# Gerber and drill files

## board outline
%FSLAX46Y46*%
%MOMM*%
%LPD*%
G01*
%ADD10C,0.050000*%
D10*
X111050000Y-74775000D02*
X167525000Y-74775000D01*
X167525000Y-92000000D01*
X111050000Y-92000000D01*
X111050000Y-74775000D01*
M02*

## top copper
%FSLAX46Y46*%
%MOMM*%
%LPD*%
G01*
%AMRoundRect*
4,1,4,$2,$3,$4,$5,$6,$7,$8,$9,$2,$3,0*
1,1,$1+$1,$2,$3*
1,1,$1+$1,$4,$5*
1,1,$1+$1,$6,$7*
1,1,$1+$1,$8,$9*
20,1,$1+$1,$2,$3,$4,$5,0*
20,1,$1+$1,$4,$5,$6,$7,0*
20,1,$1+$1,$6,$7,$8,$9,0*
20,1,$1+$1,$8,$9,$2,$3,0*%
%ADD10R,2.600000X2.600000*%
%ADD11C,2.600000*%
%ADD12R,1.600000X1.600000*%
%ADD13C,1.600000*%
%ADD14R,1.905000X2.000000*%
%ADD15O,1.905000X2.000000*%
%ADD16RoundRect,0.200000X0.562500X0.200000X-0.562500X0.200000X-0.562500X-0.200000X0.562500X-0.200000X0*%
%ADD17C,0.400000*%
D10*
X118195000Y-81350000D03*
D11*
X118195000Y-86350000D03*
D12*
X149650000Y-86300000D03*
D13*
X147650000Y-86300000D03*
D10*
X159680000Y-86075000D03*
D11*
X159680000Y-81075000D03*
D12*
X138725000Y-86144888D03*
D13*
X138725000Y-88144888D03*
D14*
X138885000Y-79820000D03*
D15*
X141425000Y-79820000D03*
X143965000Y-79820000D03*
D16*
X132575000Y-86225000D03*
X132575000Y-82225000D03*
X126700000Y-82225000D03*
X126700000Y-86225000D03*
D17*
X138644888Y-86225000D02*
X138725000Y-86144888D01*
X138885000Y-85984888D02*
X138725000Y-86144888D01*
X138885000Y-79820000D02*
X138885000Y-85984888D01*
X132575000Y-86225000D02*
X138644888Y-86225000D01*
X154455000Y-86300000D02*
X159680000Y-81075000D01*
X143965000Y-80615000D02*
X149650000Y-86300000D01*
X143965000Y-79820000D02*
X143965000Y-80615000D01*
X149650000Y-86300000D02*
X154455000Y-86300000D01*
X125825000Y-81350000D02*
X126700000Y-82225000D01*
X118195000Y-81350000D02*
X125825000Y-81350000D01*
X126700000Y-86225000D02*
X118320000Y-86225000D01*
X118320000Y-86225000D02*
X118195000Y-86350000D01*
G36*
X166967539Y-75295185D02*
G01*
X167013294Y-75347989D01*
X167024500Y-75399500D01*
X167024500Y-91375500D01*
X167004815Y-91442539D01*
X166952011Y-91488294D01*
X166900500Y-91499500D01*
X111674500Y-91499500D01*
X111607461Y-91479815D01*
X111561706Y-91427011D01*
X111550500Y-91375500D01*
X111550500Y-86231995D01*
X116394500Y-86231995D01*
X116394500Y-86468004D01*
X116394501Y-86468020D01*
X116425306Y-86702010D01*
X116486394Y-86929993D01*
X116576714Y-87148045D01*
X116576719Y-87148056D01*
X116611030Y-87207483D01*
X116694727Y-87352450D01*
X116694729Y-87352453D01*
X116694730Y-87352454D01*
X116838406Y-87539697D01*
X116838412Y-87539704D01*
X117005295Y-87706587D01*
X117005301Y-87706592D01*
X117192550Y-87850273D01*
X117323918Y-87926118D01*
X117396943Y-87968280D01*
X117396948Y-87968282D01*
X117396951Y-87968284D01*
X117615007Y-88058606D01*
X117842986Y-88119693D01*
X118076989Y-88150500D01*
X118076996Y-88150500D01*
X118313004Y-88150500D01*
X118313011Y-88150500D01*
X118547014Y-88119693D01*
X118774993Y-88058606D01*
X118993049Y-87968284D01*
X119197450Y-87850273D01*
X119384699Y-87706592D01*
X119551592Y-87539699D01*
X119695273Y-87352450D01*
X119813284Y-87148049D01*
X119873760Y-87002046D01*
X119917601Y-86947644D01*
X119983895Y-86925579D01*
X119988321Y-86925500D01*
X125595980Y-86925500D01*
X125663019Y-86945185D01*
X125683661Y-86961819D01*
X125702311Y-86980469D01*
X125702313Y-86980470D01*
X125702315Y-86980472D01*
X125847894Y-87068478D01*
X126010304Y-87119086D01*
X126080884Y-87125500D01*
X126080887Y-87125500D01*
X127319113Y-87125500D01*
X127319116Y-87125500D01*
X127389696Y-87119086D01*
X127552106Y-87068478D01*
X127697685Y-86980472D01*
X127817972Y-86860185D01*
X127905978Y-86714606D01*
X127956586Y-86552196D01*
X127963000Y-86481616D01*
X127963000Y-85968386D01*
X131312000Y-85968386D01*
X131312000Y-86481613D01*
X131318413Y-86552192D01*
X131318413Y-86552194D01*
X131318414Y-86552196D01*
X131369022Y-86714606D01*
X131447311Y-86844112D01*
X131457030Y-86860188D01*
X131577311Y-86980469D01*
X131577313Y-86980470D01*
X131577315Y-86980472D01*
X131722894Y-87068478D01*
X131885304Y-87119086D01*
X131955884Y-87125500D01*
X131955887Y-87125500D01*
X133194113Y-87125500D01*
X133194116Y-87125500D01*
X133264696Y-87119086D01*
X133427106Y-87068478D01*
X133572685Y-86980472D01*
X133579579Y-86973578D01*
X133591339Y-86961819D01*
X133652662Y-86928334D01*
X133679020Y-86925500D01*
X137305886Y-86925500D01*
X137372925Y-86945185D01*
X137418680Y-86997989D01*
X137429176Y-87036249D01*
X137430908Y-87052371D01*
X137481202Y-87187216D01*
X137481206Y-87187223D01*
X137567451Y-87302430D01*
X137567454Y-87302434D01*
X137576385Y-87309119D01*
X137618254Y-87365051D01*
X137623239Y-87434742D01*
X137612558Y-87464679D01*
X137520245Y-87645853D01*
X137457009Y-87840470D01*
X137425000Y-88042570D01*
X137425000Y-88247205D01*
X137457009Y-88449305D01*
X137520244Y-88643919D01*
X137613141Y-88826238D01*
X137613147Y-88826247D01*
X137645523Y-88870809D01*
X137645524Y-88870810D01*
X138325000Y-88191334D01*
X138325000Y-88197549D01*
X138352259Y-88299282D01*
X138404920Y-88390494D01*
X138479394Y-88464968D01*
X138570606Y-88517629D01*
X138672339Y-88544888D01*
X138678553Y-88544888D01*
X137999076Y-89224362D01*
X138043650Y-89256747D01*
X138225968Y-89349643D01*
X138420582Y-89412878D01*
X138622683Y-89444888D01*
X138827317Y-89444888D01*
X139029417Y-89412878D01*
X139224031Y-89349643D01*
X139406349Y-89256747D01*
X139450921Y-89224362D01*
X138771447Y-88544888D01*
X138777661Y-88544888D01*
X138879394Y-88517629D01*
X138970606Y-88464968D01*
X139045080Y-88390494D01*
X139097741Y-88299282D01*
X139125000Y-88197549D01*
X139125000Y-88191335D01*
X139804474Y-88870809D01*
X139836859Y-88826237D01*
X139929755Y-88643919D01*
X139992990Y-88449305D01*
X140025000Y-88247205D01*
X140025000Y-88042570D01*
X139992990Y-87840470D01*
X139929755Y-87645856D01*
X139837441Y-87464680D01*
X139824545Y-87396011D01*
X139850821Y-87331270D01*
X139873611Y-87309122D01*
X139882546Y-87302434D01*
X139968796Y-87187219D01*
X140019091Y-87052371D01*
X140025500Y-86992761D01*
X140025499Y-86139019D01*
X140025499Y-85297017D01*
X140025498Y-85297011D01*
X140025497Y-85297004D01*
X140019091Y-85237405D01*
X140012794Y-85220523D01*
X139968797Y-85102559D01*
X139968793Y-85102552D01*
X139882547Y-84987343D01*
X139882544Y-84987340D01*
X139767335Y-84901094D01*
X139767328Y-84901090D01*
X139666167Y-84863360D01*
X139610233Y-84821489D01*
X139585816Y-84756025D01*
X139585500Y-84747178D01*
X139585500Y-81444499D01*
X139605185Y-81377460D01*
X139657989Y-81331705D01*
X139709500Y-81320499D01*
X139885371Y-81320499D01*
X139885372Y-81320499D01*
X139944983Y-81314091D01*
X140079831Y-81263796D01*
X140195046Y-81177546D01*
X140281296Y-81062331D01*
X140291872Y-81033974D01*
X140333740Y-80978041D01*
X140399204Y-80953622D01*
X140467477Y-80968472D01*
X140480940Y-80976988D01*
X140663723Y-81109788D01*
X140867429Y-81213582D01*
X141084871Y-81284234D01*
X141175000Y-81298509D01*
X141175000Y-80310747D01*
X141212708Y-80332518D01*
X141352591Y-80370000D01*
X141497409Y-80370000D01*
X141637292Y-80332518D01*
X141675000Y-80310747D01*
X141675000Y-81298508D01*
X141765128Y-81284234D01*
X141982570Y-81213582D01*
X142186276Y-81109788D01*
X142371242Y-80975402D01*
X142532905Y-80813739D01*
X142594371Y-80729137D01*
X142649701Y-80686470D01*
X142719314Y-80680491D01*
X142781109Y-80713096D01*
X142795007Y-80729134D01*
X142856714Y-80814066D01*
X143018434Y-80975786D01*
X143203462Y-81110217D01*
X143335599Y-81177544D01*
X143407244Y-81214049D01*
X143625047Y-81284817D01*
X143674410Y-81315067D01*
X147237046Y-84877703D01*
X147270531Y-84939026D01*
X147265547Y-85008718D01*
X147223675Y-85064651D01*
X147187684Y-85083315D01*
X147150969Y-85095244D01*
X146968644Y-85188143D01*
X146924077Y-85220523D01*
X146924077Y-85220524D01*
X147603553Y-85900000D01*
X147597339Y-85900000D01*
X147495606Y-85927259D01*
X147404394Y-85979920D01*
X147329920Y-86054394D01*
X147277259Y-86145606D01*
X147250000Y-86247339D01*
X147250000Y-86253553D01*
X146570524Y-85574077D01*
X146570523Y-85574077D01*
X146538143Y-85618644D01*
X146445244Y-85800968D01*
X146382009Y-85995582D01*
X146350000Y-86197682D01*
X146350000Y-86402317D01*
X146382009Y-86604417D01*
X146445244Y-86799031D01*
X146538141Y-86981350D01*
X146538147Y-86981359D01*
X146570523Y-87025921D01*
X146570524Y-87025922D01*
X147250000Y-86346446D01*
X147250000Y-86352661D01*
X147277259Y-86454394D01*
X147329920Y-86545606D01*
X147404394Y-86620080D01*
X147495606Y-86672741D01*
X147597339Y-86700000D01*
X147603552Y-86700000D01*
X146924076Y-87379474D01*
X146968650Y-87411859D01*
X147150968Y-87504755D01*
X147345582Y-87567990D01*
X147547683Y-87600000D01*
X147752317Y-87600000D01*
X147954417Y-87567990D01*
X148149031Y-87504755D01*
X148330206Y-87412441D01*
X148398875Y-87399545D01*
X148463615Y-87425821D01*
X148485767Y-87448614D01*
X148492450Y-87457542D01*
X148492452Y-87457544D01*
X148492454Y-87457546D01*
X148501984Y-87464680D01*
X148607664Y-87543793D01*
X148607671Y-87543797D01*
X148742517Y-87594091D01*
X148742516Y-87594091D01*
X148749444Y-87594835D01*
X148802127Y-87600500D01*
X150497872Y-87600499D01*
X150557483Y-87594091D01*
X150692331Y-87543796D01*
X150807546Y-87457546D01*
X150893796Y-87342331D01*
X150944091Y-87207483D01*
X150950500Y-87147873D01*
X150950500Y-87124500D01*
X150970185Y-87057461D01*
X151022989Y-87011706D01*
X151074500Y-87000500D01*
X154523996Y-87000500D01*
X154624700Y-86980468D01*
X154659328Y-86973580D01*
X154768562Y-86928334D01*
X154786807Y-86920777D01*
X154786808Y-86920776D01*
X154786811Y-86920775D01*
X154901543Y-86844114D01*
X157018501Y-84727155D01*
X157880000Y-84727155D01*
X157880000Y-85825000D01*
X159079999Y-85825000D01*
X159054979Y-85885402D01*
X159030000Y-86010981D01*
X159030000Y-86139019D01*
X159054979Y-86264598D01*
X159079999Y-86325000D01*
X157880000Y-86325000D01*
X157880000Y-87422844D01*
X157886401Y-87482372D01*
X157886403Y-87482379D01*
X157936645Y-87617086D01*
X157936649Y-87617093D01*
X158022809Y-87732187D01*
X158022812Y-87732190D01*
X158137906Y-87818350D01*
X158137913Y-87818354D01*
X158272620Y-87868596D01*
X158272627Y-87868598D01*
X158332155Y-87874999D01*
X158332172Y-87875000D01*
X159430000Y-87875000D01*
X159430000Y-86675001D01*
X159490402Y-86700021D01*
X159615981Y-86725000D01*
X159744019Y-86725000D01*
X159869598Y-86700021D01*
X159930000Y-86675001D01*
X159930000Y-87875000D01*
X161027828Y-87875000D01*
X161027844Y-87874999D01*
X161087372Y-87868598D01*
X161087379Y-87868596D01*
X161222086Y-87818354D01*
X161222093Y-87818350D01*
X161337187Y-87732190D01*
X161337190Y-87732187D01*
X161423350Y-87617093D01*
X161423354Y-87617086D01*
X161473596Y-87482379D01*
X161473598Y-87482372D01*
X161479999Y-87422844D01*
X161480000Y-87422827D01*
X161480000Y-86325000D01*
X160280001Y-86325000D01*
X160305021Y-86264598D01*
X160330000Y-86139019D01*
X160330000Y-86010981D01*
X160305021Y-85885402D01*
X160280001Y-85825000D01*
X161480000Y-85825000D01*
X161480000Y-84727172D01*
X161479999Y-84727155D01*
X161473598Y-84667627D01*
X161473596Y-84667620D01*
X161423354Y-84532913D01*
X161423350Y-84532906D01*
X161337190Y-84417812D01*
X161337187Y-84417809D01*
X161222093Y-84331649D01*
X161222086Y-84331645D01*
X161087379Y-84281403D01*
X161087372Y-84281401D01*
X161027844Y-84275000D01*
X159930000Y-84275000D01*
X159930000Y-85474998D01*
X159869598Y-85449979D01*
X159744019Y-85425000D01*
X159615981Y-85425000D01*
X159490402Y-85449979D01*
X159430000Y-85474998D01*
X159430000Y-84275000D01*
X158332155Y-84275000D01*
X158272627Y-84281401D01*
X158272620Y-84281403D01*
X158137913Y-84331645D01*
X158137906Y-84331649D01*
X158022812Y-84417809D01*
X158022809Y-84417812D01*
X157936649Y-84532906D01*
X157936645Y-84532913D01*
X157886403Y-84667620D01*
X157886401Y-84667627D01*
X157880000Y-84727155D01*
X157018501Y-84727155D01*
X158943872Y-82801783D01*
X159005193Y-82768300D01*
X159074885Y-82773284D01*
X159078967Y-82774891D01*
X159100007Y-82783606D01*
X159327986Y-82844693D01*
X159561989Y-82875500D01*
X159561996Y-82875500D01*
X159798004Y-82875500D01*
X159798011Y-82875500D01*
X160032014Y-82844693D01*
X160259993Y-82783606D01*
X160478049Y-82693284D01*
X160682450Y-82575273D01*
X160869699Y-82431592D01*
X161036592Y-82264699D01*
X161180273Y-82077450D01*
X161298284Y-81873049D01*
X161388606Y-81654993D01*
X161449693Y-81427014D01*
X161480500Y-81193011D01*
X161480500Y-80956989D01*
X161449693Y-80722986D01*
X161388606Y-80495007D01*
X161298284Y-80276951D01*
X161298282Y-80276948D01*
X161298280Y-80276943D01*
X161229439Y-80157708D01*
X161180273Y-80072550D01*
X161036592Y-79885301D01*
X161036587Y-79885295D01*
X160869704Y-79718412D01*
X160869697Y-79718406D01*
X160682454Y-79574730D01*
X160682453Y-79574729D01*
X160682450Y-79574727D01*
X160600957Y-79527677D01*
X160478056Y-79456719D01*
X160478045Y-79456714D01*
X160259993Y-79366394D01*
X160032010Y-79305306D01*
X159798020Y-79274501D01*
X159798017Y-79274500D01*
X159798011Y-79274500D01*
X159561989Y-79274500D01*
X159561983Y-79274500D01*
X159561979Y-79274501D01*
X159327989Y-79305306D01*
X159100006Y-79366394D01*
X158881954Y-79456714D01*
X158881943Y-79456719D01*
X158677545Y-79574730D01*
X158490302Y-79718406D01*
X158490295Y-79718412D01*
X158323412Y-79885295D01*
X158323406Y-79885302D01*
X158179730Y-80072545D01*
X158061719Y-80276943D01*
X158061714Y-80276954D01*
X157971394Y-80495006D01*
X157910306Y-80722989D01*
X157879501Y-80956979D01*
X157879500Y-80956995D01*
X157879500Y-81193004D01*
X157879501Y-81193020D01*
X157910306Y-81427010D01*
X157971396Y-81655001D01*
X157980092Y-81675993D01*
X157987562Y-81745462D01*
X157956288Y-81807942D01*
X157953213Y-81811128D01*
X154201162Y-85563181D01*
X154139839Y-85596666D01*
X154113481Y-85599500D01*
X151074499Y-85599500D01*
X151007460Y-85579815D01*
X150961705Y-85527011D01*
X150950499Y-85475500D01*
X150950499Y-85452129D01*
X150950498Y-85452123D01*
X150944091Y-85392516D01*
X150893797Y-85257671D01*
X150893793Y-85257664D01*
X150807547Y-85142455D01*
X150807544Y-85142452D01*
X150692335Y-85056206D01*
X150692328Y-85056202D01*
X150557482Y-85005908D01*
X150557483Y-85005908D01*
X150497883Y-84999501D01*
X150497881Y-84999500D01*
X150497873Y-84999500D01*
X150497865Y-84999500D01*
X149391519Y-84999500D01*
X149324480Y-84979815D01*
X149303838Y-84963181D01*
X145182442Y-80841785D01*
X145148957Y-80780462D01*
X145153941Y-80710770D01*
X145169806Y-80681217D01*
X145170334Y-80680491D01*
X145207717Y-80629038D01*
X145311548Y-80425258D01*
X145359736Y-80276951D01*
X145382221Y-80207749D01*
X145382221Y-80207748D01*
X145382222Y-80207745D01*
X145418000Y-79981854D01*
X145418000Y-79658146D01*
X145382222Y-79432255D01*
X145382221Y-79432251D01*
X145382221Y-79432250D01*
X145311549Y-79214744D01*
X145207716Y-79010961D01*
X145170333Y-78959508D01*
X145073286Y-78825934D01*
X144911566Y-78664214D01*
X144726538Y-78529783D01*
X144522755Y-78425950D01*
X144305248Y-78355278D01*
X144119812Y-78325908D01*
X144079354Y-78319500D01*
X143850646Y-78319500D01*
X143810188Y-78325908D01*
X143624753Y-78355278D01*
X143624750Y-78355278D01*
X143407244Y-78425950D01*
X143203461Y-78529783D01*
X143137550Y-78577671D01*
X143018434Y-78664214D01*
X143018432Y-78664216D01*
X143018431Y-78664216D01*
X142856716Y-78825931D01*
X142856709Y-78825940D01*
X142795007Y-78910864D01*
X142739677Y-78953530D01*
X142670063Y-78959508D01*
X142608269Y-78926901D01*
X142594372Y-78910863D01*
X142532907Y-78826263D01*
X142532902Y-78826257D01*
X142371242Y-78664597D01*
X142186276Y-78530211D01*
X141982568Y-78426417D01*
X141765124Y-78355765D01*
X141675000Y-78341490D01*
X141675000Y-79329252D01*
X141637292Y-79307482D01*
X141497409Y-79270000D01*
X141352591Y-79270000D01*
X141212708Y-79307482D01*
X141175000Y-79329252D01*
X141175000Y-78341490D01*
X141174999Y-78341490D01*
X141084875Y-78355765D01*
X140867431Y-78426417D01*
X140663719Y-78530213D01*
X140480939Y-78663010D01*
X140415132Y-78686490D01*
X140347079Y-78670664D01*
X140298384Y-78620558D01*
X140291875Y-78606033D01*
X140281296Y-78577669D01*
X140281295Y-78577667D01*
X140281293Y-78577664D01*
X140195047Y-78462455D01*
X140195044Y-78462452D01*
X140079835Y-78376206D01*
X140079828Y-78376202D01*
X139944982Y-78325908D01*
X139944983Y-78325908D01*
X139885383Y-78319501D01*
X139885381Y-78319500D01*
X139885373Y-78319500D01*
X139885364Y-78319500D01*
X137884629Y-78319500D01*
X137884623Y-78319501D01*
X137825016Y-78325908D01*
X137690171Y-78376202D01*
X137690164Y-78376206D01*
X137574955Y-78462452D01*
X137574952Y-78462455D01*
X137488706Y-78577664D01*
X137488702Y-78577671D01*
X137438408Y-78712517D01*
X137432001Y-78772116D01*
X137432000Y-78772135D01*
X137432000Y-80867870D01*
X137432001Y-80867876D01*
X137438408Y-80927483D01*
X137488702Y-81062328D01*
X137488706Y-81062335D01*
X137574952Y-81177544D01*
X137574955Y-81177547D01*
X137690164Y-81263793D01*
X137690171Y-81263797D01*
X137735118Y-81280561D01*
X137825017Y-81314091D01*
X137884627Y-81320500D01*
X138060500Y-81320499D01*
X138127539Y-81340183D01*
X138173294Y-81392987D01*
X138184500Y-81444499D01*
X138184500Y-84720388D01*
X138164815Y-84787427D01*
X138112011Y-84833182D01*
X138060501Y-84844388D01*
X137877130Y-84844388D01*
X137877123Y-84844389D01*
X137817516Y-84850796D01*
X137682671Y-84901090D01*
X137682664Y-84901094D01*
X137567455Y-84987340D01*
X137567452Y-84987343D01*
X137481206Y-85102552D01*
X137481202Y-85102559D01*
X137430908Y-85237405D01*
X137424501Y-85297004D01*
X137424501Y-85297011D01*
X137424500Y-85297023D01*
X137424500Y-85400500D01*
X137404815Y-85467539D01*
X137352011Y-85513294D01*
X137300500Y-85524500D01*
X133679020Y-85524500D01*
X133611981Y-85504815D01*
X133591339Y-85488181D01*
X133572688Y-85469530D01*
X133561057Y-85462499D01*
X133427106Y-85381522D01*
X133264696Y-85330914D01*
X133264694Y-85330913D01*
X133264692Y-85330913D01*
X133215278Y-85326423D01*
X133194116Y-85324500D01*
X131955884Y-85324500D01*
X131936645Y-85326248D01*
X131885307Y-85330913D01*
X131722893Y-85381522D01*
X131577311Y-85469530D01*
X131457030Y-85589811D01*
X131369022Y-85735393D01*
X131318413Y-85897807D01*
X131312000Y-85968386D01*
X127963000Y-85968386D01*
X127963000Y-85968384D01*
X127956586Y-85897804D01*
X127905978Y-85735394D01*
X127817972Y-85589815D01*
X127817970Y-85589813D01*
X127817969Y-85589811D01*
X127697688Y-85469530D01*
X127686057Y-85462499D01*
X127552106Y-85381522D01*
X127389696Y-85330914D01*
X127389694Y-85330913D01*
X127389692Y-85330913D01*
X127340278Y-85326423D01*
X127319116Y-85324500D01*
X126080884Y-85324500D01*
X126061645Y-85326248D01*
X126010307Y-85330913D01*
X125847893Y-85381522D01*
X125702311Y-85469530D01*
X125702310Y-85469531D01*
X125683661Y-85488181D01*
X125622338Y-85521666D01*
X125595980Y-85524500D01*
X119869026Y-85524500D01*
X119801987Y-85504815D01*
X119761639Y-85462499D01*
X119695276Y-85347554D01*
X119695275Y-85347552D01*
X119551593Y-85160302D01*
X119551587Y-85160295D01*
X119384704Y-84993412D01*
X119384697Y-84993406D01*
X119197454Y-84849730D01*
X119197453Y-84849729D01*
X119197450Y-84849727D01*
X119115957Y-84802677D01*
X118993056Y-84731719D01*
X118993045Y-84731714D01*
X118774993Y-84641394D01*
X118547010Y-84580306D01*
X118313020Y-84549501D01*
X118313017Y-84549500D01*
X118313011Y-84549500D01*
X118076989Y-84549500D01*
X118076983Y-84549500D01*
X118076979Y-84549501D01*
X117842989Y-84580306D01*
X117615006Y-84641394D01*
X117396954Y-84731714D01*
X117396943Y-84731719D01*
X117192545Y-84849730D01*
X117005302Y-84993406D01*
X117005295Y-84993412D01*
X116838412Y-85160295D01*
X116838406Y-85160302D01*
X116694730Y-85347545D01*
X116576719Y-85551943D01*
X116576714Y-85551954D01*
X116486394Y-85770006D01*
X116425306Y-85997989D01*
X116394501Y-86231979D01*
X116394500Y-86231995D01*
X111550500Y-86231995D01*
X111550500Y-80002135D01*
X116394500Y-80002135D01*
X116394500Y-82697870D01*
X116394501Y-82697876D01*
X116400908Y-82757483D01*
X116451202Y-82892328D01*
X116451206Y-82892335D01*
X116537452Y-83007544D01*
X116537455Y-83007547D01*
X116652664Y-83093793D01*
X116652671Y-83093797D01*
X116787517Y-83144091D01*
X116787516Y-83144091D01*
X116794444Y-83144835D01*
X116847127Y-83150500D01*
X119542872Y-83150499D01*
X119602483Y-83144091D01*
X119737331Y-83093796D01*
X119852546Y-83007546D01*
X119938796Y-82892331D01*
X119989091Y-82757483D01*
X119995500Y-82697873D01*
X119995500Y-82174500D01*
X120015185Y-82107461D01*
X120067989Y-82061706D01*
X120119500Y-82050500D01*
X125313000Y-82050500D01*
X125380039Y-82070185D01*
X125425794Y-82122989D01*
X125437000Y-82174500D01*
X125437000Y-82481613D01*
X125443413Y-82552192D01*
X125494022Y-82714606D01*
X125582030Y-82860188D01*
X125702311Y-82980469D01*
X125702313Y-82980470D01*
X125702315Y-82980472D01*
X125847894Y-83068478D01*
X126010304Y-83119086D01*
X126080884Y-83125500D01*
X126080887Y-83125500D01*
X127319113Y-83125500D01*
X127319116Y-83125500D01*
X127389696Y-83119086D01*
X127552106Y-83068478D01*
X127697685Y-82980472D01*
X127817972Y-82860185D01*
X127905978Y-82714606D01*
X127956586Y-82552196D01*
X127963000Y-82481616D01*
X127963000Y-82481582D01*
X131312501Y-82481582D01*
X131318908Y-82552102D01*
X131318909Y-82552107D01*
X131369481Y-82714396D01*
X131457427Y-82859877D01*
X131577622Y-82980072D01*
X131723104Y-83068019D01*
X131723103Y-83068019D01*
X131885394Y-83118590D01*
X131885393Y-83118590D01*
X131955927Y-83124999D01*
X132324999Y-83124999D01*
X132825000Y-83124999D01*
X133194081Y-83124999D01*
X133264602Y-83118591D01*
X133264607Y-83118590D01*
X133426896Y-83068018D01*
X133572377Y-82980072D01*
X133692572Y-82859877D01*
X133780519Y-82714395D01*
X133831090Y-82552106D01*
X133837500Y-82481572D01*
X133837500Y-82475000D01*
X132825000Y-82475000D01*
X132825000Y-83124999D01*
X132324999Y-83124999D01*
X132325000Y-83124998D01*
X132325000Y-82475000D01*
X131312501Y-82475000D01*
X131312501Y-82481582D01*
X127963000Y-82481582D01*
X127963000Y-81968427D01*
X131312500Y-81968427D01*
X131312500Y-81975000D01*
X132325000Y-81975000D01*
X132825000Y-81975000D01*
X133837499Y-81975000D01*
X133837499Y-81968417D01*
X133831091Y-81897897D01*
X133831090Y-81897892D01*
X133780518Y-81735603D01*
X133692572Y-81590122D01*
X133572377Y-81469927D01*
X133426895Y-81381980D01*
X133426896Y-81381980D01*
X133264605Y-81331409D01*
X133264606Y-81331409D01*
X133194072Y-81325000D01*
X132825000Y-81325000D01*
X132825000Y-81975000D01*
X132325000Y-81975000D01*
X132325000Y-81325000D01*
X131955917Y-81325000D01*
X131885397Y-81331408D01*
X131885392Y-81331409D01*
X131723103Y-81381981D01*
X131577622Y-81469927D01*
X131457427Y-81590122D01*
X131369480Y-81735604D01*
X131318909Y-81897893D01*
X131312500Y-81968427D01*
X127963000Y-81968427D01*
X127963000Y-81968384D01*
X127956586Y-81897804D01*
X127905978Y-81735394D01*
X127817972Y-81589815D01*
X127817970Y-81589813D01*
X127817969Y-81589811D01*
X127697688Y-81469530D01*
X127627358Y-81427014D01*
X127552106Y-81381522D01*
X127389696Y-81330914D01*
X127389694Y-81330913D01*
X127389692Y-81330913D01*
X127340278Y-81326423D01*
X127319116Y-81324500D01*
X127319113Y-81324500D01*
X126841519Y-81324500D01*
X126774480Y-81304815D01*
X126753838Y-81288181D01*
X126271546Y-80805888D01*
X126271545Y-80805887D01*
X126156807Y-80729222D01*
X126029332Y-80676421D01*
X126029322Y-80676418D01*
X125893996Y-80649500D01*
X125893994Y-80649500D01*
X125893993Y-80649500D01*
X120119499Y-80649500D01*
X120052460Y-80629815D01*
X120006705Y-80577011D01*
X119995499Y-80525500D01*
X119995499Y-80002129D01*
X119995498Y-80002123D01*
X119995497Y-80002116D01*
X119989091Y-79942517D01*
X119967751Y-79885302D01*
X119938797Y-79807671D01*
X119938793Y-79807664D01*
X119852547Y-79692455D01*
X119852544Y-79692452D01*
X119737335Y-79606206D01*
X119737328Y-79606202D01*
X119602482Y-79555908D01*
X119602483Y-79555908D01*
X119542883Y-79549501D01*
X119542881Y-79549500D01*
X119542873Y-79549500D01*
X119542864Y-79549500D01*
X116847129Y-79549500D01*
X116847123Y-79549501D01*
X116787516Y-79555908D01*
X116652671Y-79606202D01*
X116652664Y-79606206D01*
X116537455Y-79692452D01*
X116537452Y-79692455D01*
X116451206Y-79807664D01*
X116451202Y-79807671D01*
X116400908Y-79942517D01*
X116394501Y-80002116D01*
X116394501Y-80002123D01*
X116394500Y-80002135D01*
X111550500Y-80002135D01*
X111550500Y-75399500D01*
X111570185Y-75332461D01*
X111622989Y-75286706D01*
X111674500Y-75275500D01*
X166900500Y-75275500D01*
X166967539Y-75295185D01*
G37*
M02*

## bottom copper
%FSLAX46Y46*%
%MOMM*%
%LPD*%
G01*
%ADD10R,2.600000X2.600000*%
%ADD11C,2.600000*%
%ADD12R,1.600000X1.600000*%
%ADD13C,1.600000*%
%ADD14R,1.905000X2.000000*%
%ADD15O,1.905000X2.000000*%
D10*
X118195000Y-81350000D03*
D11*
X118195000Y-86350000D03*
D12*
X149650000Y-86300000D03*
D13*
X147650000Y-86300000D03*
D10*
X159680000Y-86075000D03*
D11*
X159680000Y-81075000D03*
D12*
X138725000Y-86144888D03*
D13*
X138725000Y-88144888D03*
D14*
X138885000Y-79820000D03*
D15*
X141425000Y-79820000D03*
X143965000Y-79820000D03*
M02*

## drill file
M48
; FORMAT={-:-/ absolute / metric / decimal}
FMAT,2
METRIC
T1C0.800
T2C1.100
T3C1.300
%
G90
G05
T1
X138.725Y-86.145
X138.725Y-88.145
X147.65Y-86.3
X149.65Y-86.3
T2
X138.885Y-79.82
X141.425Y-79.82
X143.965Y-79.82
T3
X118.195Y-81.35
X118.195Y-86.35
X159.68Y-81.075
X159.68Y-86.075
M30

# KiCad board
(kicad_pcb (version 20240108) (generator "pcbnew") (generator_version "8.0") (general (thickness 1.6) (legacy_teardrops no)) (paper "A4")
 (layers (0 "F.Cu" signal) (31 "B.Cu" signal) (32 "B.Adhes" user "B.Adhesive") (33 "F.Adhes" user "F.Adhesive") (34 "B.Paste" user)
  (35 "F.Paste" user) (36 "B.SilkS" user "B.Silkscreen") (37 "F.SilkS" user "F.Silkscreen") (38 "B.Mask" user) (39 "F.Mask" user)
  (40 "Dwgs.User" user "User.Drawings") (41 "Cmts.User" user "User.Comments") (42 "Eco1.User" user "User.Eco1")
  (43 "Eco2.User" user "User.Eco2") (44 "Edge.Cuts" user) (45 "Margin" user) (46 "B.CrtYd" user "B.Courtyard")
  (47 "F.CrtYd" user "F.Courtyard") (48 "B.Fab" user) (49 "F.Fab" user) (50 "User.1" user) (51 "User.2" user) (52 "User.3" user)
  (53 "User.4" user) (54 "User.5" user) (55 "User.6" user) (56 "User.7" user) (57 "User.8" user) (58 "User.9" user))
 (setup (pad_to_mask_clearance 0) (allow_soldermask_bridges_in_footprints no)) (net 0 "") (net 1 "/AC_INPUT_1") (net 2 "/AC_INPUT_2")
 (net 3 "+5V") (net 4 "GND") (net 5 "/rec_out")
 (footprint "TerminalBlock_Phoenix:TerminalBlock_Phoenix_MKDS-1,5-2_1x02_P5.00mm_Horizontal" (layer "F.Cu") (at 118.195 81.35 -90)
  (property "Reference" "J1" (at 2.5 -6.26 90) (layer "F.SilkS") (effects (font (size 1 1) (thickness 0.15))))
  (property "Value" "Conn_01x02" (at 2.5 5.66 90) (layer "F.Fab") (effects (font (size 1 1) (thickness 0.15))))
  (pad "1" thru_hole rect (at 0 0 270) (size 2.6 2.6) (drill 1.3) (layers "*.Cu" "*.Mask") (remove_unused_layers no) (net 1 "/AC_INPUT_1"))
  (pad "2" thru_hole circle (at 5 0 270) (size 2.6 2.6) (drill 1.3) (layers "*.Cu" "*.Mask") (remove_unused_layers no) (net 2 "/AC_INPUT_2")))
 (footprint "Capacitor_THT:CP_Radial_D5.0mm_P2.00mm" (layer "F.Cu") (at 149.65 86.3 180)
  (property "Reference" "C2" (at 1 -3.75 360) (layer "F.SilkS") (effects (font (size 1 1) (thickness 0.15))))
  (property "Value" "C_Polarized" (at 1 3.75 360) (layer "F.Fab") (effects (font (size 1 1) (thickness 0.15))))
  (pad "1" thru_hole rect (at 0 0 180) (size 1.6 1.6) (drill 0.8) (layers "*.Cu" "*.Mask") (remove_unused_layers no) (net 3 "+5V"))
  (pad "2" thru_hole circle (at 2 0 180) (size 1.6 1.6) (drill 0.8) (layers "*.Cu" "*.Mask") (remove_unused_layers no) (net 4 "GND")))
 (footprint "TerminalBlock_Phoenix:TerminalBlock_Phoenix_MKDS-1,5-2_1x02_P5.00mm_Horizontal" (layer "F.Cu") (at 159.68 86.075 90)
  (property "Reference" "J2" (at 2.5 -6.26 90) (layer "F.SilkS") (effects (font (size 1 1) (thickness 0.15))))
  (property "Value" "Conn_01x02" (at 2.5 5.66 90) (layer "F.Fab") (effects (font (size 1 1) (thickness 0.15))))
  (pad "1" thru_hole rect (at 0 0 90) (size 2.6 2.6) (drill 1.3) (layers "*.Cu" "*.Mask") (remove_unused_layers no) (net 4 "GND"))
  (pad "2" thru_hole circle (at 5 0 90) (size 2.6 2.6) (drill 1.3) (layers "*.Cu" "*.Mask") (remove_unused_layers no) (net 3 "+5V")))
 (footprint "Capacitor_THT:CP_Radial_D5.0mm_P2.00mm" (layer "F.Cu") (at 138.725 86.144888 -90)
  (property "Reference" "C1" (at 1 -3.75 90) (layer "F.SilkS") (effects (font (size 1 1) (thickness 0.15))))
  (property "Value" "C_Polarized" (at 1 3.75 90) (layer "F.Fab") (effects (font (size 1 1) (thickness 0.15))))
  (pad "1" thru_hole rect (at 0 0 270) (size 1.6 1.6) (drill 0.8) (layers "*.Cu" "*.Mask") (remove_unused_layers no) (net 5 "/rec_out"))
  (pad "2" thru_hole circle (at 2 0 270) (size 1.6 1.6) (drill 0.8) (layers "*.Cu" "*.Mask") (remove_unused_layers no) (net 4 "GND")))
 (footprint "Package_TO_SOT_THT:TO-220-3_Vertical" (layer "F.Cu") (at 138.885 79.82)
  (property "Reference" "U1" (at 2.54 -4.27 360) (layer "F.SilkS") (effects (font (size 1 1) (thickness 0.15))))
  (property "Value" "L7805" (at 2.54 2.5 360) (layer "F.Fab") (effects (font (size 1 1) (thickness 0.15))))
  (pad "1" thru_hole rect (at 0 0) (size 1.905 2) (drill 1.1) (layers "*.Cu" "*.Mask") (remove_unused_layers no) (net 5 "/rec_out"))
  (pad "2" thru_hole oval (at 2.54 0) (size 1.905 2) (drill 1.1) (layers "*.Cu" "*.Mask") (remove_unused_layers no) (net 4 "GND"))
  (pad "3" thru_hole oval (at 5.08 0) (size 1.905 2) (drill 1.1) (layers "*.Cu" "*.Mask") (remove_unused_layers no) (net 3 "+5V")))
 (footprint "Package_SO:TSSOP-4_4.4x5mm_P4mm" (layer "F.Cu") (at 129.6375 84.225 180)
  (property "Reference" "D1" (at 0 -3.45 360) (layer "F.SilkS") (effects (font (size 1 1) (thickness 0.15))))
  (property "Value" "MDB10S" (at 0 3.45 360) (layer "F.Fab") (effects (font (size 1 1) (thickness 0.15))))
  (pad "1" smd roundrect (at -2.9375 -2 180) (size 1.525 0.8) (layers "F.Cu" "F.Paste" "F.Mask") (roundrect_rratio 0.25) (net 5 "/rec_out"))
  (pad "2" smd roundrect (at -2.9375 2 180) (size 1.525 0.8) (layers "F.Cu" "F.Paste" "F.Mask") (roundrect_rratio 0.25) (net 4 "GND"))
  (pad "3" smd roundrect (at 2.9375 2 180) (size 1.525 0.8) (layers "F.Cu" "F.Paste" "F.Mask") (roundrect_rratio 0.25) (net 1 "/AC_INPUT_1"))
  (pad "4" smd roundrect (at 2.9375 -2 180) (size 1.525 0.8) (layers "F.Cu" "F.Paste" "F.Mask") (roundrect_rratio 0.25)
   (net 2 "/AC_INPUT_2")))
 (gr_rect (start 111.05 74.775) (end 167.525 92) (stroke (width 0.05) (type default)) (fill none) (layer "Edge.Cuts"))
 (segment (start 138.644888 86.225) (end 138.725 86.144888) (width 0.4) (layer "F.Cu") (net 5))
 (segment (start 138.885 85.984888) (end 138.725 86.144888) (width 0.4) (layer "F.Cu") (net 5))
 (segment (start 138.885 79.82) (end 138.885 85.984888) (width 0.4) (layer "F.Cu") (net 5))
 (segment (start 132.575 86.225) (end 138.644888 86.225) (width 0.4) (layer "F.Cu") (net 5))
 (segment (start 154.455 86.3) (end 159.68 81.075) (width 0.4) (layer "F.Cu") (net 3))
 (segment (start 143.965 80.615) (end 149.65 86.3) (width 0.4) (layer "F.Cu") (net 3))
 (segment (start 143.965 79.82) (end 143.965 80.615) (width 0.4) (layer "F.Cu") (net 3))
 (segment (start 149.65 86.3) (end 154.455 86.3) (width 0.4) (layer "F.Cu") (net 3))
 (segment (start 125.825 81.35) (end 126.7 82.225) (width 0.4) (layer "F.Cu") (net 1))
 (segment (start 118.195 81.35) (end 125.825 81.35) (width 0.4) (layer "F.Cu") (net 1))
 (segment (start 126.7 86.225) (end 118.32 86.225) (width 0.4) (layer "F.Cu") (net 2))
 (segment (start 118.32 86.225) (end 118.195 86.35) (width 0.4) (layer "F.Cu") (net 2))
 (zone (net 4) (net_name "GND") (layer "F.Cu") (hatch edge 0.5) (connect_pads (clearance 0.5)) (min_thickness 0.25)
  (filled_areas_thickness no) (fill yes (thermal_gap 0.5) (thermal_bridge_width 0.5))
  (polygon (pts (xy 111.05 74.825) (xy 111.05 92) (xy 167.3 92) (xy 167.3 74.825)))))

